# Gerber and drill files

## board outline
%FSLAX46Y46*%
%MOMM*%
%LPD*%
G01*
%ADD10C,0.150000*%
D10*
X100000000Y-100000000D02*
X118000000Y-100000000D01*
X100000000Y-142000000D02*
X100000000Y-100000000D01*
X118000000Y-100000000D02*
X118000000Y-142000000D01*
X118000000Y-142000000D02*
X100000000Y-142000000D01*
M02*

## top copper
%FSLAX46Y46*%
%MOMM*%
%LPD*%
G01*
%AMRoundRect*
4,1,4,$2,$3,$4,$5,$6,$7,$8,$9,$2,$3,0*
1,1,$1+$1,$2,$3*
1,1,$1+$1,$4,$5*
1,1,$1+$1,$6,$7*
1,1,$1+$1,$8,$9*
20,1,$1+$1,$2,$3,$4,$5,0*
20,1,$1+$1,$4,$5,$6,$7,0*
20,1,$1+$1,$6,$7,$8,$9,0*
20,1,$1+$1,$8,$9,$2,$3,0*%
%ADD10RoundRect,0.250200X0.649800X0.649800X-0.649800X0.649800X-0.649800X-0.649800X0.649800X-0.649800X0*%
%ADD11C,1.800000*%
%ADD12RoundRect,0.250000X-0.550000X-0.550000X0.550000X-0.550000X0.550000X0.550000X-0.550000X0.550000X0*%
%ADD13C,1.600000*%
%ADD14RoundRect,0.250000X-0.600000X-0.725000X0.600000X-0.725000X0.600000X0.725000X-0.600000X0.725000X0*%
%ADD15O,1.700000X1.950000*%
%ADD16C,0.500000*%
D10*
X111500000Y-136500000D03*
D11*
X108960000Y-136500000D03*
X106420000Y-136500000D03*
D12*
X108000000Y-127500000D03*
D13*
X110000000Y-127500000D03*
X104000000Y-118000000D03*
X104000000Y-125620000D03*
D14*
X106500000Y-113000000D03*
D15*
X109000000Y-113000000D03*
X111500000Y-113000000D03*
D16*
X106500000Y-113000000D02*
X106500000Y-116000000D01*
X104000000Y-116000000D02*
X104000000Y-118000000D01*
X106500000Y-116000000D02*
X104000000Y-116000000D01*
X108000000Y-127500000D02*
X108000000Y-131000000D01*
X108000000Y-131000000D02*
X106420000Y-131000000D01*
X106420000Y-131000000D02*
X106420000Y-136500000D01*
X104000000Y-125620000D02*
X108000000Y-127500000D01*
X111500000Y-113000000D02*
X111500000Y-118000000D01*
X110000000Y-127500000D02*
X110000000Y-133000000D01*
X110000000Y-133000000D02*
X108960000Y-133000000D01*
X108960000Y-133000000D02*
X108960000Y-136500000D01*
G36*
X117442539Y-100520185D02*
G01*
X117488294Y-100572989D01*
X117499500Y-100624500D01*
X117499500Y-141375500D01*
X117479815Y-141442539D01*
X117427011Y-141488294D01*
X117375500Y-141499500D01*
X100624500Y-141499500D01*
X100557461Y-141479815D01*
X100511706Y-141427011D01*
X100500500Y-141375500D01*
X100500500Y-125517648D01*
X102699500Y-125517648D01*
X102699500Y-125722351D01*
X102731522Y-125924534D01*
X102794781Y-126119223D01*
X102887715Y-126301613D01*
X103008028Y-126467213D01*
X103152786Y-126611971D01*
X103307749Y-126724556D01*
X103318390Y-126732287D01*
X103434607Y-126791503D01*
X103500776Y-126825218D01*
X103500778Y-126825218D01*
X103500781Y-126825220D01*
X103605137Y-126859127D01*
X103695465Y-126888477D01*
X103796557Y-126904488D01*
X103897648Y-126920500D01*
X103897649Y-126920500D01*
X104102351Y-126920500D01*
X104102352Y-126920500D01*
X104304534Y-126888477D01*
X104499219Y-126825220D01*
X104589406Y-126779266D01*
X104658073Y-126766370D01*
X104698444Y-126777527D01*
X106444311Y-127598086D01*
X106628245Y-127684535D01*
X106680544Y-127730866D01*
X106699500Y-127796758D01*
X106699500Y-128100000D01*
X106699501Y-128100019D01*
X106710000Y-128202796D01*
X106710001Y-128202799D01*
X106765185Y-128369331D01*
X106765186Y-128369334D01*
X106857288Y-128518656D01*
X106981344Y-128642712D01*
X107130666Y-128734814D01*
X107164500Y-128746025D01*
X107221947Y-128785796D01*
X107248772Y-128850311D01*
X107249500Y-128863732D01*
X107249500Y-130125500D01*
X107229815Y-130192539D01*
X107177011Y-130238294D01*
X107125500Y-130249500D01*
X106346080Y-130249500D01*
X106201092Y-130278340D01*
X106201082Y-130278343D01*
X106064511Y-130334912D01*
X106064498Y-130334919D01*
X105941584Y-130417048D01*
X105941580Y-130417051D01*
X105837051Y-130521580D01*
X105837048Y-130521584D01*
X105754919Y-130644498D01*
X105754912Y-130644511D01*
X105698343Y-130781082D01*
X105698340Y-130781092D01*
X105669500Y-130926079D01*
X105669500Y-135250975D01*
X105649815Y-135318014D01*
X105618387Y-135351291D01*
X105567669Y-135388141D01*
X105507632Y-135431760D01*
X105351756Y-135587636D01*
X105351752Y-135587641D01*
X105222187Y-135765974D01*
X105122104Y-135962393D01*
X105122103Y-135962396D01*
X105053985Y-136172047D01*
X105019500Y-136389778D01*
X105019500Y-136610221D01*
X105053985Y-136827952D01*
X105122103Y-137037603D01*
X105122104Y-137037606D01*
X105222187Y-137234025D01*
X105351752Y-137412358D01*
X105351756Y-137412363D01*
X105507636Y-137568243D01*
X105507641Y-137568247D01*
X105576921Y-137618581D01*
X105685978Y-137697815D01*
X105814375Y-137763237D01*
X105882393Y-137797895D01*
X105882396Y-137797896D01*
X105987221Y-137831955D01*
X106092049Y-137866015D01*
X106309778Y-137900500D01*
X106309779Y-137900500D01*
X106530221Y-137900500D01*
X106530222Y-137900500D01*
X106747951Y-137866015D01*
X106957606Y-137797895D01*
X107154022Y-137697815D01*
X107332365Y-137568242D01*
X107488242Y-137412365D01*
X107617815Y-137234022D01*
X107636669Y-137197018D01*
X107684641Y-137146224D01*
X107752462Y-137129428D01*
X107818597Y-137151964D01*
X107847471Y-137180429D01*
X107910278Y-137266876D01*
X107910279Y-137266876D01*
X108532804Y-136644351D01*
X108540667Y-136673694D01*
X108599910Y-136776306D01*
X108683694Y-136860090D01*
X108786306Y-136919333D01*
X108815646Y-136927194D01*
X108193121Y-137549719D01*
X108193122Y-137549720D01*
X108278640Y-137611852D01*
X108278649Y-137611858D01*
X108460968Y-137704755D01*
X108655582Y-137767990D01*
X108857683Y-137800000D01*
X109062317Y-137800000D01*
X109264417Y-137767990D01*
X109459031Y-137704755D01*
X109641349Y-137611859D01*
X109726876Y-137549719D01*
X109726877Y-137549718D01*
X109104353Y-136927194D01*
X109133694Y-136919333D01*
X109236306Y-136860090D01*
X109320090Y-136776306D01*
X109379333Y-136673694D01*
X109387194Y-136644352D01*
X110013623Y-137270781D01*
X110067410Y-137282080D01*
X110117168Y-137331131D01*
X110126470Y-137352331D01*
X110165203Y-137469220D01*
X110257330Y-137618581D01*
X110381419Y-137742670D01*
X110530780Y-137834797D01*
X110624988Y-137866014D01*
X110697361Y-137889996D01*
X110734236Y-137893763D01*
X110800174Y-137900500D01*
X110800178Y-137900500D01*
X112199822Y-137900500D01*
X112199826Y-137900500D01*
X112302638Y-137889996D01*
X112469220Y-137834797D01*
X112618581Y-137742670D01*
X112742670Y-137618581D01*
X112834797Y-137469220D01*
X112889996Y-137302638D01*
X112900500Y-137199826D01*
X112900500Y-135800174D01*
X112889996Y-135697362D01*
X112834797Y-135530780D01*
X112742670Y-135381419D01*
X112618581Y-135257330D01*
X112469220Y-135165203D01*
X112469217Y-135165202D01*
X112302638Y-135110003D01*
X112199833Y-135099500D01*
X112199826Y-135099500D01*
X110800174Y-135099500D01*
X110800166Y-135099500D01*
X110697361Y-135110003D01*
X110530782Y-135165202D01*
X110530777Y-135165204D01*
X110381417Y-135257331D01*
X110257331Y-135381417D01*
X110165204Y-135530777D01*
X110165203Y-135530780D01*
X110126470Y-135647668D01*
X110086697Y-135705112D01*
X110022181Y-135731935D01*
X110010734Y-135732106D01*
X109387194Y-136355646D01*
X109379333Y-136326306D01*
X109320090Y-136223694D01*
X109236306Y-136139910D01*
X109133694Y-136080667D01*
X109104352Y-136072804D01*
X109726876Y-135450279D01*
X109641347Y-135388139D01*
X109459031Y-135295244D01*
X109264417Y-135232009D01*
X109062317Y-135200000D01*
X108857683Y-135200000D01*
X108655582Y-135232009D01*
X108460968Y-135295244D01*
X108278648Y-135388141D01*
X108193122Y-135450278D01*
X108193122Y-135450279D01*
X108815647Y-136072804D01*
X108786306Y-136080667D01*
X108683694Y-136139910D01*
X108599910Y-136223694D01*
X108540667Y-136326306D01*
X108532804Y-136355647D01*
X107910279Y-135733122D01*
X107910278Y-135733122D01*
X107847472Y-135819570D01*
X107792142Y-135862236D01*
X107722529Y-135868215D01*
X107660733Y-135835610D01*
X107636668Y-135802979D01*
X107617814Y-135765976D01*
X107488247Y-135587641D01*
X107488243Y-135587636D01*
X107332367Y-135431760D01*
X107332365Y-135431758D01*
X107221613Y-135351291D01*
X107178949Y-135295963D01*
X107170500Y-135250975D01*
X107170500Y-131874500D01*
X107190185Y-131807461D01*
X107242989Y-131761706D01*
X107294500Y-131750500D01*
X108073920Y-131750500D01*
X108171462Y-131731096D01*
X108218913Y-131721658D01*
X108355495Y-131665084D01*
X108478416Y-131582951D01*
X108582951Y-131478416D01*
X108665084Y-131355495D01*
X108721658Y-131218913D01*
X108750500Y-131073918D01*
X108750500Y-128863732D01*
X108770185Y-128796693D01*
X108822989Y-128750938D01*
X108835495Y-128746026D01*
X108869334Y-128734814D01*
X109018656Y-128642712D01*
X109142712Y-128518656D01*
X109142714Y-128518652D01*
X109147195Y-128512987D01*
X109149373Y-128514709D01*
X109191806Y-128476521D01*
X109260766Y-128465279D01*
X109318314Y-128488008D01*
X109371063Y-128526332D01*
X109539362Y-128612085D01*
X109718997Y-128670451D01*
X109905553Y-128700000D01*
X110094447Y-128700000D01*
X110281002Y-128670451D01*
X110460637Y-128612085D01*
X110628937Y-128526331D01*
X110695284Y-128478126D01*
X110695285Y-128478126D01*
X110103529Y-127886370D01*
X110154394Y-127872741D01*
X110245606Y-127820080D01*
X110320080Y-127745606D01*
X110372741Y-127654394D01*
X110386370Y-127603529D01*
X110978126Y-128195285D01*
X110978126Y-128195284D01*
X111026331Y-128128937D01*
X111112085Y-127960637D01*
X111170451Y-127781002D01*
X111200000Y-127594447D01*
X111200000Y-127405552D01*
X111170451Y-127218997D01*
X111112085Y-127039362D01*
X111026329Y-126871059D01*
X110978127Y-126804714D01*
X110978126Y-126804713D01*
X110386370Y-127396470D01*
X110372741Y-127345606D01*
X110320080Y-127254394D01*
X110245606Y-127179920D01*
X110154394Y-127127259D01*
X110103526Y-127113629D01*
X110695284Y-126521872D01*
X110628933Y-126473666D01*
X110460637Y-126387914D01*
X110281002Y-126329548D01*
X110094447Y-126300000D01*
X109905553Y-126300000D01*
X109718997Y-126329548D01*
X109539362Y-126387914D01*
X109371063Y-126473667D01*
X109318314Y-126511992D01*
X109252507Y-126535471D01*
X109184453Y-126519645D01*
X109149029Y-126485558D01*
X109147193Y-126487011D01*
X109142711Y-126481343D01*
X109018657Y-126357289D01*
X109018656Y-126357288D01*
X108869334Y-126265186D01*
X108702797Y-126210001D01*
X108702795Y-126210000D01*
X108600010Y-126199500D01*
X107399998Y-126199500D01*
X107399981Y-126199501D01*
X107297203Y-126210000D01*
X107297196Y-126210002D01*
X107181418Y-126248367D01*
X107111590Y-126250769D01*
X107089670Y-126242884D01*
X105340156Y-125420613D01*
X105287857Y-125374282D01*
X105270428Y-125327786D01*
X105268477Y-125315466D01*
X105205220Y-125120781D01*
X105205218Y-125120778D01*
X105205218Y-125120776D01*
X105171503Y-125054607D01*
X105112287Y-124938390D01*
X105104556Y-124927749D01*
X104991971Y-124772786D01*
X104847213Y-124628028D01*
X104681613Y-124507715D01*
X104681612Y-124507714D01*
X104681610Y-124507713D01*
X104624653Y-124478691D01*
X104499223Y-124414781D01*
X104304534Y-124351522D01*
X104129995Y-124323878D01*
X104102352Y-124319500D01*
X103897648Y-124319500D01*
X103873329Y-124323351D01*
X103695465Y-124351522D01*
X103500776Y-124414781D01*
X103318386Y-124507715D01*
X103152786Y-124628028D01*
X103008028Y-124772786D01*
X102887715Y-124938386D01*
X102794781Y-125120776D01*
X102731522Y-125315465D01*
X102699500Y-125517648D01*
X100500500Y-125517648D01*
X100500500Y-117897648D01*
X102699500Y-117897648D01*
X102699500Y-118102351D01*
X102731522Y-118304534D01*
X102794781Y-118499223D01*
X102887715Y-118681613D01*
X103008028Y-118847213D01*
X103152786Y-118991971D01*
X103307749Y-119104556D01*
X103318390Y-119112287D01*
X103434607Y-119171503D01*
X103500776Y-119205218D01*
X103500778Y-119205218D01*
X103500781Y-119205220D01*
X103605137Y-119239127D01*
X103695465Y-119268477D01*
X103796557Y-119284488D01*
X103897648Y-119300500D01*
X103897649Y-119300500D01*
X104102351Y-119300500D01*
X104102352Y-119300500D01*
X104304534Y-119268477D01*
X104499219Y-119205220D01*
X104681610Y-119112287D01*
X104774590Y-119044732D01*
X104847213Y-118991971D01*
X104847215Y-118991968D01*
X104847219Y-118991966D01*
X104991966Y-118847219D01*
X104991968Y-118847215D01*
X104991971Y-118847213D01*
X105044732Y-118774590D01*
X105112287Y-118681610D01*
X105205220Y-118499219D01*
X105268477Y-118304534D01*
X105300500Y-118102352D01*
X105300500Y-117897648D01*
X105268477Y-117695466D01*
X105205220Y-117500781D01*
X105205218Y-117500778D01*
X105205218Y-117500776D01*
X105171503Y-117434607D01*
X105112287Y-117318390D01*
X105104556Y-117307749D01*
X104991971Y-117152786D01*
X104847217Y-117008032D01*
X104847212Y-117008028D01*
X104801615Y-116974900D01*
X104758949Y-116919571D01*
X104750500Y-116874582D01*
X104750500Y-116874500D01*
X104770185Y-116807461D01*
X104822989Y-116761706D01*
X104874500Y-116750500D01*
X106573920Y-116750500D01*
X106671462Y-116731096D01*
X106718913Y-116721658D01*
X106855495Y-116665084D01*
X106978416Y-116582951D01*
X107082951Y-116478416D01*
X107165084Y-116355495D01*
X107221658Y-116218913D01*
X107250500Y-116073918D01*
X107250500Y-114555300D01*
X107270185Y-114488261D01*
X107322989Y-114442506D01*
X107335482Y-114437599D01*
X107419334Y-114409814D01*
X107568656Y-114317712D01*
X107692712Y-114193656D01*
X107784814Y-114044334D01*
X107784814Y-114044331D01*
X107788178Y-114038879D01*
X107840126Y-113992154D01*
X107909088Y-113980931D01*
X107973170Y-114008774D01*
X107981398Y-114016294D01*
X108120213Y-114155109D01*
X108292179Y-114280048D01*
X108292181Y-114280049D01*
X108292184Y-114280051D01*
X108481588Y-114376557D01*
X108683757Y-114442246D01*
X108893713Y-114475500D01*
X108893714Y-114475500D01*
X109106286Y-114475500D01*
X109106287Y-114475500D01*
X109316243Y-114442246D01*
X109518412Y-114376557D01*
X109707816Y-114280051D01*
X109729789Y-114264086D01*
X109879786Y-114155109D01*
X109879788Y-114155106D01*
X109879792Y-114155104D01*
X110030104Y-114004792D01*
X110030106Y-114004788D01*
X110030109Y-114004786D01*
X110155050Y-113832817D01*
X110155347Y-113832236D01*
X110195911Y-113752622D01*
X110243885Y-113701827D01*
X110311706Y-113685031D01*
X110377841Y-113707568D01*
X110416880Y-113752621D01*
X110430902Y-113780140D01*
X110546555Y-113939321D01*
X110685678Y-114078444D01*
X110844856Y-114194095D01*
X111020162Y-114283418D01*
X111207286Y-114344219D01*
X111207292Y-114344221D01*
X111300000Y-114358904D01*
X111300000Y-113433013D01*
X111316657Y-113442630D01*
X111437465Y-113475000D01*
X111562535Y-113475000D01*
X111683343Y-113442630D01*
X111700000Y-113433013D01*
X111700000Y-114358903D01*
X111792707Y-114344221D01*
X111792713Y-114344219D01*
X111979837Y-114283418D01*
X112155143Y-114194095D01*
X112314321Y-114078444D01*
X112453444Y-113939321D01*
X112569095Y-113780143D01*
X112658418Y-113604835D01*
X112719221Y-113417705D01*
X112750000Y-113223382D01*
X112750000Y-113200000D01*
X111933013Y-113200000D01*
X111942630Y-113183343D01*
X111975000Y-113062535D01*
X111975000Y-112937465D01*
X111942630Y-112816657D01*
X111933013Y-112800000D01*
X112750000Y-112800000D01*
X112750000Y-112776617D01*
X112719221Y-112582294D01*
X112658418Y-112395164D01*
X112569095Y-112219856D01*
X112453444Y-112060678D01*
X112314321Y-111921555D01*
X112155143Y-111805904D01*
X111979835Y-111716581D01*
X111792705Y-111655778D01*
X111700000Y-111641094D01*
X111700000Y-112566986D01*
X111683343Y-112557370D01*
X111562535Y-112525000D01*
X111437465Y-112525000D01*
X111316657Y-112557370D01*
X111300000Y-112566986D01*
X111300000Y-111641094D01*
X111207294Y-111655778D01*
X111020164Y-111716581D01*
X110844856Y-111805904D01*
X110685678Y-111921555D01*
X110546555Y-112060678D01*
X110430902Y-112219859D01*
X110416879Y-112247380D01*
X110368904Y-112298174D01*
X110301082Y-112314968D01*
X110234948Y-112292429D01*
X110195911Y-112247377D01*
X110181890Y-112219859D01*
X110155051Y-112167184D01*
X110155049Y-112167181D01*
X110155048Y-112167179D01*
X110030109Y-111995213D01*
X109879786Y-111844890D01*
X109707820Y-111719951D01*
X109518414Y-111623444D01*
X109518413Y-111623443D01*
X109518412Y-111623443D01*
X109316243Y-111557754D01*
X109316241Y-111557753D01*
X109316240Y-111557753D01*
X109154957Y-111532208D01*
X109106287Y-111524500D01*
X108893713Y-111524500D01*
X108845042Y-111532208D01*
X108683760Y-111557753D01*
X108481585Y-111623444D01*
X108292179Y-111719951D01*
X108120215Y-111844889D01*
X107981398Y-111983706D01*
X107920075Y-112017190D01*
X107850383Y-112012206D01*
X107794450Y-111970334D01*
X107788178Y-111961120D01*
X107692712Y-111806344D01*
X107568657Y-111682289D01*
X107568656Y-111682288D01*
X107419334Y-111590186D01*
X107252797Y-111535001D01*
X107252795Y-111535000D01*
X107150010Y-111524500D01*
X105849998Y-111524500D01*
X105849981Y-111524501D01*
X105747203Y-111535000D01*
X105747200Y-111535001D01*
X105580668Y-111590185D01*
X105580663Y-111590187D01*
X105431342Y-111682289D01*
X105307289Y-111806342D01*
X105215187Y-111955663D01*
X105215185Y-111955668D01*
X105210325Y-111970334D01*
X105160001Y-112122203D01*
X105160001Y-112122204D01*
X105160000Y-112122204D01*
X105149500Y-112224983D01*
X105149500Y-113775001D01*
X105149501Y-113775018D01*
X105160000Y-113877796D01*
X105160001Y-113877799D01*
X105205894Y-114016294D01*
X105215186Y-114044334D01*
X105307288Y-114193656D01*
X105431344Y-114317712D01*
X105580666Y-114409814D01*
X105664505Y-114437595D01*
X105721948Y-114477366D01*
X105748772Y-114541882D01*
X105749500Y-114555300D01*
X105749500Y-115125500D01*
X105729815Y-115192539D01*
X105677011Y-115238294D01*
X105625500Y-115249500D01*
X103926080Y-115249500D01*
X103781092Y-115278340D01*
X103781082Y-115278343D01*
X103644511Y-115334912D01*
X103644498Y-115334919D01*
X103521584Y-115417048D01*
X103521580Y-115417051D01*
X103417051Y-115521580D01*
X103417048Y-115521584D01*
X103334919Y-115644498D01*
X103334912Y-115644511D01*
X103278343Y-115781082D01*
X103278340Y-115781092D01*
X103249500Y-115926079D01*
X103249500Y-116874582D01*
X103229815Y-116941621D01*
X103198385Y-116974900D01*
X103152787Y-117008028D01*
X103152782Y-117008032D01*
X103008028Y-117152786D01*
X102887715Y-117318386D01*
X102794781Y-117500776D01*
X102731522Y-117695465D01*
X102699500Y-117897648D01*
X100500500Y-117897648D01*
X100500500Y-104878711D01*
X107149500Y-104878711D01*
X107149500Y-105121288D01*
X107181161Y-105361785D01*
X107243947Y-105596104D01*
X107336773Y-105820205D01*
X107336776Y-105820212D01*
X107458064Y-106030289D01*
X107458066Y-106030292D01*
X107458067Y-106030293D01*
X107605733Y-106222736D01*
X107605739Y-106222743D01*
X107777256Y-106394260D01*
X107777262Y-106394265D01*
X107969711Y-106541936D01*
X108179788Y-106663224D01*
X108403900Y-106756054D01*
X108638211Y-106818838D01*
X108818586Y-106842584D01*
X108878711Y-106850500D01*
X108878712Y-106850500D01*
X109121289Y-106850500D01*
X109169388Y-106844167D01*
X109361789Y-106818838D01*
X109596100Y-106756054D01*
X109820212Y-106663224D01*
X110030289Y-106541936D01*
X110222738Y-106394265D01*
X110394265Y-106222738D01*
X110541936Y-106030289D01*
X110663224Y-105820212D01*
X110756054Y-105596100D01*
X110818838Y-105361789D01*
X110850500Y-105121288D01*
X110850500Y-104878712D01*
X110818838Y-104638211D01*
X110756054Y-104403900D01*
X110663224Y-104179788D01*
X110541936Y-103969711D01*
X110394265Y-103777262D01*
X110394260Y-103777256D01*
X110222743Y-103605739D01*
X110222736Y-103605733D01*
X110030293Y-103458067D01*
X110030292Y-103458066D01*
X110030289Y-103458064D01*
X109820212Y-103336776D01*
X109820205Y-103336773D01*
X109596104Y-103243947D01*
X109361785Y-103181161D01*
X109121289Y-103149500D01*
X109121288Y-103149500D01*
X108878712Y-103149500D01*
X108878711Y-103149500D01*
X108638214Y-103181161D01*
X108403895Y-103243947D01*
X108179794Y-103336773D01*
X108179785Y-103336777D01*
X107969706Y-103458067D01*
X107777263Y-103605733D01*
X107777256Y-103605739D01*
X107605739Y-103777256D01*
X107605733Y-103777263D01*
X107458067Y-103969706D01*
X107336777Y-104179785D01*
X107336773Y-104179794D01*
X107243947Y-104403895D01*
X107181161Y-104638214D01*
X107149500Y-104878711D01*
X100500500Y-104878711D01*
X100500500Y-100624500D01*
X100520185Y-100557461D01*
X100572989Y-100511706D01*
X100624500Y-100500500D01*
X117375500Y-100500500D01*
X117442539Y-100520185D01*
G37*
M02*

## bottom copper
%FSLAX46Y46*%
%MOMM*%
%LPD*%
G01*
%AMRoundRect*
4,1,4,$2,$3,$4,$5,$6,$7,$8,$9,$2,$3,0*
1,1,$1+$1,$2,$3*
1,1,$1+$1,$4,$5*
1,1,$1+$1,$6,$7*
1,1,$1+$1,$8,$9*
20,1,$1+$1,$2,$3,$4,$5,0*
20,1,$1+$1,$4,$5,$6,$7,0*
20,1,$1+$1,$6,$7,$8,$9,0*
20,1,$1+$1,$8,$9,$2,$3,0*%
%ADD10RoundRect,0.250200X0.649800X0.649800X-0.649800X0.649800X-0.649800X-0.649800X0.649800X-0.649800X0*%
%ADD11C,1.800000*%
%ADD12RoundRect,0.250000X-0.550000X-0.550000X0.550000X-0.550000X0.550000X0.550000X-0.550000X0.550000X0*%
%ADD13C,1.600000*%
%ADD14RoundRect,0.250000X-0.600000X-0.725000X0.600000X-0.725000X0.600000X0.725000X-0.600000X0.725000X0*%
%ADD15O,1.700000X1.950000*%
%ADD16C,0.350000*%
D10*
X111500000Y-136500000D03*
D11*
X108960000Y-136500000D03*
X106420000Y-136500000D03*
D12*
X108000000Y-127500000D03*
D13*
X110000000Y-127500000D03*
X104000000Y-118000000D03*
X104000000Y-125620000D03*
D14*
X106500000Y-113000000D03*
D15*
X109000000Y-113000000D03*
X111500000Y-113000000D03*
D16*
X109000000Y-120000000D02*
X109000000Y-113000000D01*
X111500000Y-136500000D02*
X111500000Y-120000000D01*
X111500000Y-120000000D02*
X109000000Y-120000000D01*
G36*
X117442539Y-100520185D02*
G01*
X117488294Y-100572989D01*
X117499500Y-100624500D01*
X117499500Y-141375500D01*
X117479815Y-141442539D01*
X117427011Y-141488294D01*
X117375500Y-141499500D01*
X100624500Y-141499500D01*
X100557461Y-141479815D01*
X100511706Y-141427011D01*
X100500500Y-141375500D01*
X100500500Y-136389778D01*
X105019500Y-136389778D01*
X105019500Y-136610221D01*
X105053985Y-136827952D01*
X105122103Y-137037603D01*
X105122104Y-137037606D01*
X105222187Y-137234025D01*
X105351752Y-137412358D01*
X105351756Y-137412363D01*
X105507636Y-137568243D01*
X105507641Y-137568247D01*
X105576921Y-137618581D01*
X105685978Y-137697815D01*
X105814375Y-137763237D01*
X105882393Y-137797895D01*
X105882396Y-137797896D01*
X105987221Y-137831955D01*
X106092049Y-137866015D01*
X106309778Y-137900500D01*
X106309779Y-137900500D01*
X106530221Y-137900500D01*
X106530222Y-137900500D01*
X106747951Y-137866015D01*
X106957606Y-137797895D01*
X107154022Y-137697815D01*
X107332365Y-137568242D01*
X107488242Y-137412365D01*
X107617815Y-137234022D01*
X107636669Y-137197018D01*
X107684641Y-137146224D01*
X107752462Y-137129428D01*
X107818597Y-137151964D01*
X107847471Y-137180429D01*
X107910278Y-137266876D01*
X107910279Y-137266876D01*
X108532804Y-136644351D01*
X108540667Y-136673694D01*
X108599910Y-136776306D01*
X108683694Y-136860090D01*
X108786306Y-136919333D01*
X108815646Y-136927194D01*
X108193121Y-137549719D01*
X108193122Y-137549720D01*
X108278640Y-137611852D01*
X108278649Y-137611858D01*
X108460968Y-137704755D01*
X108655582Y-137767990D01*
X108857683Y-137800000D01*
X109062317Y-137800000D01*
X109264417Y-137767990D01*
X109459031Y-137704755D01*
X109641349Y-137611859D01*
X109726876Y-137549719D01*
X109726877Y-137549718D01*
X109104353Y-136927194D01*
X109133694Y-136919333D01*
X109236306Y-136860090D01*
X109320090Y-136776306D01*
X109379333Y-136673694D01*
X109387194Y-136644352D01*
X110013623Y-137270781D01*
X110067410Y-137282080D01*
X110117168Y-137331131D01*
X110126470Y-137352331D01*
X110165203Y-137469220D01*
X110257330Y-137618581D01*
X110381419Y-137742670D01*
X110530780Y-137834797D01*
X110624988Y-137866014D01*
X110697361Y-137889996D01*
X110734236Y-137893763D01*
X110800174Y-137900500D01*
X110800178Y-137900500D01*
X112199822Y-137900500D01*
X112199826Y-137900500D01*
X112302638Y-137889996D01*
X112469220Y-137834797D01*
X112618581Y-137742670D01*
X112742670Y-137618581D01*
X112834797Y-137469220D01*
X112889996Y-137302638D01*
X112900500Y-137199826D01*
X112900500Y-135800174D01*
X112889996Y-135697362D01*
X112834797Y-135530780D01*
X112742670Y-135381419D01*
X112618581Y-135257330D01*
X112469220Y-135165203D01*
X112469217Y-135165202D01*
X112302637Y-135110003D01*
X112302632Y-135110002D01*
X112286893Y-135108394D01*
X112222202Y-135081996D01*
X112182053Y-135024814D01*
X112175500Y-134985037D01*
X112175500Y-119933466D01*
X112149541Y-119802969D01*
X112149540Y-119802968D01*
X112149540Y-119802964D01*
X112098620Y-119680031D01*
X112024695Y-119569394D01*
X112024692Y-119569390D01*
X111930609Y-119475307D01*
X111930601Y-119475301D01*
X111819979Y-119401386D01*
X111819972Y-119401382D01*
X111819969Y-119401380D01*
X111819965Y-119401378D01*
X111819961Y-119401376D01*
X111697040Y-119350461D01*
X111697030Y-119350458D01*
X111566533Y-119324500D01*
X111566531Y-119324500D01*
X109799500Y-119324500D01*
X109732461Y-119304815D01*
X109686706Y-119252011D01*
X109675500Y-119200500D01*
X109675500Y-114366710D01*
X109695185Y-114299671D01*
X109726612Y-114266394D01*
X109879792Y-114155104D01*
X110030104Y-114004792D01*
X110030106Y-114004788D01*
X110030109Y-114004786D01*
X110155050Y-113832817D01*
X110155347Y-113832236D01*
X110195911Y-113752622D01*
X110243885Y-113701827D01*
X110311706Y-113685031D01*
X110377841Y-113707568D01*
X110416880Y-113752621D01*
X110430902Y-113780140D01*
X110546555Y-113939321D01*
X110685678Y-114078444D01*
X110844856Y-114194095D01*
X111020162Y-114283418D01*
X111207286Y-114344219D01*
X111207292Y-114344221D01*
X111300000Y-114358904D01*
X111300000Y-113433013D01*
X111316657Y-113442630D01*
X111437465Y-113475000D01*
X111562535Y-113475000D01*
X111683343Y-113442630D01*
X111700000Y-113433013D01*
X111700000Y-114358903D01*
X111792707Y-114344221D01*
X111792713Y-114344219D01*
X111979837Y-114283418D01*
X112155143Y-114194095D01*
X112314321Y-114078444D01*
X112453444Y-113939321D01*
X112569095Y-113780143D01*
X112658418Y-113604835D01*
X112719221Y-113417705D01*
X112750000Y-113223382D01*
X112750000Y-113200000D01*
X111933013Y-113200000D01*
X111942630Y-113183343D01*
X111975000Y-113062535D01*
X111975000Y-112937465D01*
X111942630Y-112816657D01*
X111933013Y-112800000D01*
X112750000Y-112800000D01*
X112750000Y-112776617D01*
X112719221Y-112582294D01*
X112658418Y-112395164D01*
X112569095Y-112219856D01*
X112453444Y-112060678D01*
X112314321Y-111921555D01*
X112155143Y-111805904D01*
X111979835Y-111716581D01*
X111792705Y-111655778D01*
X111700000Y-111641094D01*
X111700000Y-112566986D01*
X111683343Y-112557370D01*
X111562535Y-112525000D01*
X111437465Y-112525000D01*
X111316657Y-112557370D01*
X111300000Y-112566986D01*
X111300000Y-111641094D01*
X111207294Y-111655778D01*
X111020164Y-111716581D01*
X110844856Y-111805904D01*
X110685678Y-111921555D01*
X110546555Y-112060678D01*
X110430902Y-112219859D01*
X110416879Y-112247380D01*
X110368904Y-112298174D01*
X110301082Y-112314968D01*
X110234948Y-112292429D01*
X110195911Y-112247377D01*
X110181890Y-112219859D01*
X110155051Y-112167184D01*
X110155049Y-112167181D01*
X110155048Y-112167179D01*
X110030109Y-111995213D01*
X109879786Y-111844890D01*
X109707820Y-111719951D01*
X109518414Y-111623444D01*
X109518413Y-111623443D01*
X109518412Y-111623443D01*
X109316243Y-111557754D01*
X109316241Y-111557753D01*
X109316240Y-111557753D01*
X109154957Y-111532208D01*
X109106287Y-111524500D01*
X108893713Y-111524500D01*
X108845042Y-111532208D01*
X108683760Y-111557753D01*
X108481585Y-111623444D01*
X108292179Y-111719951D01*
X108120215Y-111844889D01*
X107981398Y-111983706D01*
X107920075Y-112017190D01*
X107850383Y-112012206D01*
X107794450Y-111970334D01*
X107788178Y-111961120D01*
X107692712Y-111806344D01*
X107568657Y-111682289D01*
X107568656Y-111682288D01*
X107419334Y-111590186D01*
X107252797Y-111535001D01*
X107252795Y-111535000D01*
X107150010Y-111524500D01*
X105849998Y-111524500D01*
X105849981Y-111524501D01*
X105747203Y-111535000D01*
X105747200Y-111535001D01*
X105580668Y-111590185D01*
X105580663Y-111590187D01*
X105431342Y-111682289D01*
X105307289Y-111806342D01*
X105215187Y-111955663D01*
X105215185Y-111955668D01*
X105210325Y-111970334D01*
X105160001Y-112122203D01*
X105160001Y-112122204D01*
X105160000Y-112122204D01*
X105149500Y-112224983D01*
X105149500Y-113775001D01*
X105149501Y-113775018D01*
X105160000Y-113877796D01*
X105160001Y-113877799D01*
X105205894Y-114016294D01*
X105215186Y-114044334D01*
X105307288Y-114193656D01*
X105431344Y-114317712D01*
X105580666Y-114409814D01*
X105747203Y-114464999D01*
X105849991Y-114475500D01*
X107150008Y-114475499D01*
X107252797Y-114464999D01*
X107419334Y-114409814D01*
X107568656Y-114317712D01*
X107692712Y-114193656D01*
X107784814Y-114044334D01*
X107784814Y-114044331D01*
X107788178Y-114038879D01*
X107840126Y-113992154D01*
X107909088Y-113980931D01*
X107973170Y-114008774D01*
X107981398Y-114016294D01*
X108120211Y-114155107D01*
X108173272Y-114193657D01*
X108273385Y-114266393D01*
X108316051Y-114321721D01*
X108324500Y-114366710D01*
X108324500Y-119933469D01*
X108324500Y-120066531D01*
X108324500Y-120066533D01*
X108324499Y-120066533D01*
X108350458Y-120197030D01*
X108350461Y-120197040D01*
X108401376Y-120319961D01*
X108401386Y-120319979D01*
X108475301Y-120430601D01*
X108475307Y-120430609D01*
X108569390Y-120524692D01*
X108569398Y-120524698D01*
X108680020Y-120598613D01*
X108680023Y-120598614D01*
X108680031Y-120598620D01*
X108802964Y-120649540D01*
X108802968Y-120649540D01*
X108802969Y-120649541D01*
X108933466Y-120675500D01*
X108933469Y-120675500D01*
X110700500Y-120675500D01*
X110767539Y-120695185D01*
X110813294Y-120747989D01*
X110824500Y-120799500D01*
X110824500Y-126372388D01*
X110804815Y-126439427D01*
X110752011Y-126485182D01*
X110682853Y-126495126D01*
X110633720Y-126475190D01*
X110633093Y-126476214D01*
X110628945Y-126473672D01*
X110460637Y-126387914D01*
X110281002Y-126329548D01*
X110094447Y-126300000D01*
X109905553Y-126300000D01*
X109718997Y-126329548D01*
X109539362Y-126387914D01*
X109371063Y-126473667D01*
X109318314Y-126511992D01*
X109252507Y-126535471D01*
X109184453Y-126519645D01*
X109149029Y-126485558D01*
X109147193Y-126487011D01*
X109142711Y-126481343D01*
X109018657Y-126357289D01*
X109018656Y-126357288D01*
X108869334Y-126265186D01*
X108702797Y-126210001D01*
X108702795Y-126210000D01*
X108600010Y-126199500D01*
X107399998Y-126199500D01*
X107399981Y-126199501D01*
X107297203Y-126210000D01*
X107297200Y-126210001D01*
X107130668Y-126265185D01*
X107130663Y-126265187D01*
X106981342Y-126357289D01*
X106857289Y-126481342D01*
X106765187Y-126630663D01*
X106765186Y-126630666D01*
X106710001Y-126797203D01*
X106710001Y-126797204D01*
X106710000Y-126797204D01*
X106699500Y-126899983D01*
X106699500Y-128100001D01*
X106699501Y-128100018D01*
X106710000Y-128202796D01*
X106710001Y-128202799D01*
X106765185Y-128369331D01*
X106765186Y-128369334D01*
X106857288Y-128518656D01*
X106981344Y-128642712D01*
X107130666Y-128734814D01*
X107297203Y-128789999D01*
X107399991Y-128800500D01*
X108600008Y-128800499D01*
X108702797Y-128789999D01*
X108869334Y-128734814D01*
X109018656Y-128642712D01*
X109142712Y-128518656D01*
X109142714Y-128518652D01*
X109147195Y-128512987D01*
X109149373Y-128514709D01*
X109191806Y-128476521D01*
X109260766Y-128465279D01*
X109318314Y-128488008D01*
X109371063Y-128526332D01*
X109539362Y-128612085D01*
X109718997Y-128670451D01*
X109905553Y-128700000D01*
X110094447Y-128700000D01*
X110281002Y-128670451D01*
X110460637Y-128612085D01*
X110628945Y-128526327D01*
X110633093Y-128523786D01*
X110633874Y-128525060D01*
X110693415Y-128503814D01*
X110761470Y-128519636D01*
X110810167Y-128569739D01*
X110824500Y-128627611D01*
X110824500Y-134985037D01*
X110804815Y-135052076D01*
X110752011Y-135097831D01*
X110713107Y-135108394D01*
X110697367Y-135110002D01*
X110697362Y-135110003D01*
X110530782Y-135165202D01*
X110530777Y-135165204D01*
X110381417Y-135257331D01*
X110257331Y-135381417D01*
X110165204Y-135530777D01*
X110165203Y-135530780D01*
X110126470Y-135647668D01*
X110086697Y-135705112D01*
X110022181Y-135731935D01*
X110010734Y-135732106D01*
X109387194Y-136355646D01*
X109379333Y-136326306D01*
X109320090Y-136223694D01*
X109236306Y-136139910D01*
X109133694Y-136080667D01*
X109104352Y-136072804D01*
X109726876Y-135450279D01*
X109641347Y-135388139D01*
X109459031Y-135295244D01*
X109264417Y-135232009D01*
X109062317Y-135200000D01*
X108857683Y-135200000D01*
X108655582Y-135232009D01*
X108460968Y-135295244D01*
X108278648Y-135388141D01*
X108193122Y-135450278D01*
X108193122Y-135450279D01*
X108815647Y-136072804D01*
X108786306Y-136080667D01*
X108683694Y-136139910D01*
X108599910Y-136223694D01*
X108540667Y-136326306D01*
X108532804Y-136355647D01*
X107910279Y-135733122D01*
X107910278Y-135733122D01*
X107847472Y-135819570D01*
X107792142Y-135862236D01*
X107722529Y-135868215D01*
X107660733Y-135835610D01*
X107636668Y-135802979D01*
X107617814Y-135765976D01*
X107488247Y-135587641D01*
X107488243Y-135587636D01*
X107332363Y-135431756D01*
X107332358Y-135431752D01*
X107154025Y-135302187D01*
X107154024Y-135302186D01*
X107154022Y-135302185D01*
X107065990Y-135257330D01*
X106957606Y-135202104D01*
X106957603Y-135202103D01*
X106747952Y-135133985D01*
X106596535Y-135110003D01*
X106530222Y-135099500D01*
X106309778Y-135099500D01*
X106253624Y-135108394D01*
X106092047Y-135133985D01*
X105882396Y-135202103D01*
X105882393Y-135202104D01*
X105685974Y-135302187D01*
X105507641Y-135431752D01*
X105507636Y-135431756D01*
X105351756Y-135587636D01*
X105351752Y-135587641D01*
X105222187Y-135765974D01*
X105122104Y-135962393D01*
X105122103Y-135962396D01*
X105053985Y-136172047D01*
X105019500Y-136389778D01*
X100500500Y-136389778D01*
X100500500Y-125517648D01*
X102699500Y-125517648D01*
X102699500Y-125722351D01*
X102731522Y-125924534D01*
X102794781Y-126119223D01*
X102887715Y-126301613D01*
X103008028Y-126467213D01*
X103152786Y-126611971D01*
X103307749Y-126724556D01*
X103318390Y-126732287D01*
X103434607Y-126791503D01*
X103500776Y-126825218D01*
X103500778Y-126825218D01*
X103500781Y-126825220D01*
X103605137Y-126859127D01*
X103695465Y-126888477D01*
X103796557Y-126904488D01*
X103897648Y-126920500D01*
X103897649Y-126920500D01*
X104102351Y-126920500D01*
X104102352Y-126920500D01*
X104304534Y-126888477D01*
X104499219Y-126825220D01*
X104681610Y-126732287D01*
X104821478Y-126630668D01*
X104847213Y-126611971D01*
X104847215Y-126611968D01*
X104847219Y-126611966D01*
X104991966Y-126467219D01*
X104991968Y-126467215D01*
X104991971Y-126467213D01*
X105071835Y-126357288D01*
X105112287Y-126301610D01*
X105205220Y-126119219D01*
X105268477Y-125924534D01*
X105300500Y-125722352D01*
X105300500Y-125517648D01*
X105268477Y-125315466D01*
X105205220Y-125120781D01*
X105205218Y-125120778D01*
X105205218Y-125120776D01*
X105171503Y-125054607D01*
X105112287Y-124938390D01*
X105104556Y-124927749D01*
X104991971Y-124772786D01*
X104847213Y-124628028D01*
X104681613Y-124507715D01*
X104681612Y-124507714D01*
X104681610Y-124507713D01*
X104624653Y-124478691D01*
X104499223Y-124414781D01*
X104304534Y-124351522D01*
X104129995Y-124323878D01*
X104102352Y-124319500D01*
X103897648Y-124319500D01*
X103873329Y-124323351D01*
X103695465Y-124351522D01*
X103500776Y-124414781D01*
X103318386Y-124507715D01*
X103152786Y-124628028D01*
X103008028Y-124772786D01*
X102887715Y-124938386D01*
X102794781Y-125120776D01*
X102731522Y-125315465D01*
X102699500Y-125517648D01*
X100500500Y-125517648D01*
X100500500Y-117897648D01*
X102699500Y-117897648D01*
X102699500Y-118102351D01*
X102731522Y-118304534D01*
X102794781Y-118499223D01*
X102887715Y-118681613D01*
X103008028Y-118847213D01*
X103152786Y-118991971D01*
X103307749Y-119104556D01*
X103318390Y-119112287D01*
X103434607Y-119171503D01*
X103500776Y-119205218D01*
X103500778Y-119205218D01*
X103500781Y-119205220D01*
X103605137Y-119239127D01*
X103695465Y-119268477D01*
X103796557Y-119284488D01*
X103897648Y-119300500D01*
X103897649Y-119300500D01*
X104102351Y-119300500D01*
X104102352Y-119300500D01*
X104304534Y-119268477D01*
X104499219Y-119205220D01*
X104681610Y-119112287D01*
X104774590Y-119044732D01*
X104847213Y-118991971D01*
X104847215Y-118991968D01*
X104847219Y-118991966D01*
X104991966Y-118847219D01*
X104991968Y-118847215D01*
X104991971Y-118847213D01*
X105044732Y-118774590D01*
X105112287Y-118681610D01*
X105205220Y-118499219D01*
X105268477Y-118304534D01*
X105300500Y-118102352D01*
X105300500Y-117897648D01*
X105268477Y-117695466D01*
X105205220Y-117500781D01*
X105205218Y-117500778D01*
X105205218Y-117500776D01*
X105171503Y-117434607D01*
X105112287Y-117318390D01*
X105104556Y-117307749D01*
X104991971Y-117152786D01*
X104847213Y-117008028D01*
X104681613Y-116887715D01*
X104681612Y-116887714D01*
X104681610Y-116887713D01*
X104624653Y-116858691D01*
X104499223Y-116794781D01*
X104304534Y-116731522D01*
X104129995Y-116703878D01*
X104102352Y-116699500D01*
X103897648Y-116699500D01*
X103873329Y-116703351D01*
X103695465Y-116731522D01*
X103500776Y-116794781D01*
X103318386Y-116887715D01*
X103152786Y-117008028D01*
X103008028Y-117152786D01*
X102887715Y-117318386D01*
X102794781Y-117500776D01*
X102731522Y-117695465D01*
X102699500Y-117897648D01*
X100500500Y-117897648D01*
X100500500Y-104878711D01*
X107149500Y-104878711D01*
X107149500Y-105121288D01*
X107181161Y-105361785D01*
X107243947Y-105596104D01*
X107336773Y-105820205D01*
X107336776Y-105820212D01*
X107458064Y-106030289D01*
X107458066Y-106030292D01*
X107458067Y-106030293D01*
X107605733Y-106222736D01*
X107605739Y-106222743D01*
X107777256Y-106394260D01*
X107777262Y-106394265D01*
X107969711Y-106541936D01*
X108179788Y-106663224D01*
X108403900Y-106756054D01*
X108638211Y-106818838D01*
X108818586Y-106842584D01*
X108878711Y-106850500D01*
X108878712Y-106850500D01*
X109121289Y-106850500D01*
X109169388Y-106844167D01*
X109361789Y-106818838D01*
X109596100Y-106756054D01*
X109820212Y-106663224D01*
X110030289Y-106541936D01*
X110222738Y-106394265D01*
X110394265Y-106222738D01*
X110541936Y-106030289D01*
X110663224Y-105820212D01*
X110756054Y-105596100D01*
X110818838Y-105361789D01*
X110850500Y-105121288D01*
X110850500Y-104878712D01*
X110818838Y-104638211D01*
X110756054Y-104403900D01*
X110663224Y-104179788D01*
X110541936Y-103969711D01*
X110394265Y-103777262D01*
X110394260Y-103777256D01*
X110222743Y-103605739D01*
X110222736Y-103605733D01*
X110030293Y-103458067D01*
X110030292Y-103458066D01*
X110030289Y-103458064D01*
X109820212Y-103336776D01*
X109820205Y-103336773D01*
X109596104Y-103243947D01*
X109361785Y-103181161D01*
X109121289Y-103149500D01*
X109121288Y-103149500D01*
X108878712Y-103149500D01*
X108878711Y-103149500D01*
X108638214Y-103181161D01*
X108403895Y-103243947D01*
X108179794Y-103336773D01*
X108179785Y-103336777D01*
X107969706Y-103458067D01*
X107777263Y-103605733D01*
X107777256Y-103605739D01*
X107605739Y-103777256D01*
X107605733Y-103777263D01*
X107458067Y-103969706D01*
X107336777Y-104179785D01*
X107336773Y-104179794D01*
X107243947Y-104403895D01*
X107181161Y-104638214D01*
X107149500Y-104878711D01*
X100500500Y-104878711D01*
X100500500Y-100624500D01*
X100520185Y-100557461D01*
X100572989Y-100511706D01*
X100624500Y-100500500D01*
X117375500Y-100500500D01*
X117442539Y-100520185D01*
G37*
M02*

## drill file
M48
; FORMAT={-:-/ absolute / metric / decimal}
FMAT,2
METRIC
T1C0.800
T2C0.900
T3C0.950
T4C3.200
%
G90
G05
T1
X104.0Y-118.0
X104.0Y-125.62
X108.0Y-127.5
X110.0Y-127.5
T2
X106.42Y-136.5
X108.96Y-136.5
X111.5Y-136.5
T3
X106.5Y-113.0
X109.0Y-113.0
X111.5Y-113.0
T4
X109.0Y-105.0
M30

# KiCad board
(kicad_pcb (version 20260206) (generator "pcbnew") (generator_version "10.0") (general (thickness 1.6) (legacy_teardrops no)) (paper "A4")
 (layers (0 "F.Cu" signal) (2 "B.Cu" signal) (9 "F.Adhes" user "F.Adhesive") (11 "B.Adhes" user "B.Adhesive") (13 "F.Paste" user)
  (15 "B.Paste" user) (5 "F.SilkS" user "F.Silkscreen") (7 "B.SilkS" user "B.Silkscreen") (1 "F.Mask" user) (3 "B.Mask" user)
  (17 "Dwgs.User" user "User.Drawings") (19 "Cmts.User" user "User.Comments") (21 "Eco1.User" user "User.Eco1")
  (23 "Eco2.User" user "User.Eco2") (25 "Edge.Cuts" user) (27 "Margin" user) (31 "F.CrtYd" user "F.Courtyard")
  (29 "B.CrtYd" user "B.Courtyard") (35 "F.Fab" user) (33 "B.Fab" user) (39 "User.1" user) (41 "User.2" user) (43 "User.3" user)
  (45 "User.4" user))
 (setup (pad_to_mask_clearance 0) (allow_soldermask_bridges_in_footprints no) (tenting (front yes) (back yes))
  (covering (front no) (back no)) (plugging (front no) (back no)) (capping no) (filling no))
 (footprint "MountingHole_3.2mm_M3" (layer "F.Cu") (at 109 105)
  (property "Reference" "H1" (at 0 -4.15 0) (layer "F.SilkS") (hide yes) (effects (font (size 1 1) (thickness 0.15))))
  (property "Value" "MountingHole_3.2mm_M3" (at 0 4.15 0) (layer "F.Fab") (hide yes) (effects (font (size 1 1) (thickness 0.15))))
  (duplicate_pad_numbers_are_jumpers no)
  (pad "" np_thru_hole circle (at 0 0) (size 3.2 3.2) (drill 3.2) (layers "*.Cu" "*.Mask")))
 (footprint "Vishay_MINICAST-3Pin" (layer "F.Cu") (at 111.5 136.5 180)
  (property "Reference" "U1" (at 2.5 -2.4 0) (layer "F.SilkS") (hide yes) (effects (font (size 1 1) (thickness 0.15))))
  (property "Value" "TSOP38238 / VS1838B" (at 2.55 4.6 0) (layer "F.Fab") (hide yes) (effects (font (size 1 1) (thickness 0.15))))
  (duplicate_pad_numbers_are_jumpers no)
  (pad "1" thru_hole roundrect (at 0 0 180) (size 1.8 1.8) (drill 0.9) (layers "*.Cu" "*.Mask") (remove_unused_layers no)
   (roundrect_rratio 0.139) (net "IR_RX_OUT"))
  (pad "2" thru_hole circle (at 2.54 0 180) (size 1.8 1.8) (drill 0.9) (layers "*.Cu" "*.Mask") (remove_unused_layers no) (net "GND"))
  (pad "3" thru_hole circle (at 5.08 0 180) (size 1.8 1.8) (drill 0.9) (layers "*.Cu" "*.Mask") (remove_unused_layers no) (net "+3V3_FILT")))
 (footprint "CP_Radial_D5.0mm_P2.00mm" (layer "F.Cu") (at 108 127.5)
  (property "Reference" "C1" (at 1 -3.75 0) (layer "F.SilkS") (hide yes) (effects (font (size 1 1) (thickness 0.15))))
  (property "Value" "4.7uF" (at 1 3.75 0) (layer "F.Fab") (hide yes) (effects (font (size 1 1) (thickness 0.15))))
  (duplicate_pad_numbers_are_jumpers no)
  (pad "1" thru_hole roundrect (at 0 0) (size 1.6 1.6) (drill 0.8) (layers "*.Cu" "*.Mask") (remove_unused_layers no)
   (roundrect_rratio 0.15625) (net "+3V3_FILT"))
  (pad "2" thru_hole circle (at 2 0) (size 1.6 1.6) (drill 0.8) (layers "*.Cu" "*.Mask") (remove_unused_layers no) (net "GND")))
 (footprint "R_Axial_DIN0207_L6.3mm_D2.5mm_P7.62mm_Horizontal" (layer "F.Cu") (at 104 118 -90)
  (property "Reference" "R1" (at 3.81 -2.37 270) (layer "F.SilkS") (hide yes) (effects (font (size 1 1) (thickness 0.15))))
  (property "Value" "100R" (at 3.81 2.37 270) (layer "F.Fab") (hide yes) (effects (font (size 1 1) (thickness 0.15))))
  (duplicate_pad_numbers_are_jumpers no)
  (pad "1" thru_hole circle (at 0 0 270) (size 1.6 1.6) (drill 0.8) (layers "*.Cu" "*.Mask") (remove_unused_layers no) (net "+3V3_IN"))
  (pad "2" thru_hole circle (at 7.62 0 270) (size 1.6 1.6) (drill 0.8) (layers "*.Cu" "*.Mask") (remove_unused_layers no) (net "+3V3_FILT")))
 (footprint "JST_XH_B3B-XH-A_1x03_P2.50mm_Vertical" (layer "F.Cu") (at 106.5 113)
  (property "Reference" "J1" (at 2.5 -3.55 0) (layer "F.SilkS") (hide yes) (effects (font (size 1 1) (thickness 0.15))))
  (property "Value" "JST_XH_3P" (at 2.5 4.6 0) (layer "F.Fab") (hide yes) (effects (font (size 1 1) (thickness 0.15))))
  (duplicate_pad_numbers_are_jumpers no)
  (pad "1" thru_hole roundrect (at 0 0) (size 1.7 1.95) (drill 0.95) (layers "*.Cu" "*.Mask") (remove_unused_layers no)
   (roundrect_rratio 0.147059) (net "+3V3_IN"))
  (pad "2" thru_hole oval (at 2.5 0) (size 1.7 1.95) (drill 0.95) (layers "*.Cu" "*.Mask") (remove_unused_layers no) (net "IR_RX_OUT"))
  (pad "3" thru_hole oval (at 5 0) (size 1.7 1.95) (drill 0.95) (layers "*.Cu" "*.Mask") (remove_unused_layers no) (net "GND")))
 (gr_line (start 100 100) (end 118 100) (stroke (width 0.15) (type default)) (layer "Edge.Cuts"))
 (gr_line (start 100 142) (end 100 100) (stroke (width 0.15) (type default)) (layer "Edge.Cuts"))
 (gr_line (start 118 100) (end 118 142) (stroke (width 0.15) (type default)) (layer "Edge.Cuts"))
 (gr_line (start 118 142) (end 100 142) (stroke (width 0.15) (type default)) (layer "Edge.Cuts"))
 (segment (start 106.5 113) (end 106.5 116) (width 0.5) (layer "F.Cu") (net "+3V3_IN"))
 (segment (start 104 116) (end 104 118) (width 0.5) (layer "F.Cu") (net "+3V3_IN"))
 (segment (start 106.5 116) (end 104 116) (width 0.5) (layer "F.Cu") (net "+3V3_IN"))
 (segment (start 108 127.5) (end 108 131) (width 0.5) (layer "F.Cu") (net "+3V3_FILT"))
 (segment (start 108 131) (end 106.42 131) (width 0.5) (layer "F.Cu") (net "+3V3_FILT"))
 (segment (start 106.42 131) (end 106.42 136.5) (width 0.5) (layer "F.Cu") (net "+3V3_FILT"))
 (segment (start 104 125.62) (end 108 127.5) (width 0.5) (layer "F.Cu") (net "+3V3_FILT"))
 (segment (start 109 120) (end 109 113) (width 0.35) (layer "B.Cu") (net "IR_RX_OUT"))
 (segment (start 111.5 136.5) (end 111.5 120) (width 0.35) (layer "B.Cu") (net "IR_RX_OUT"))
 (segment (start 111.5 120) (end 109 120) (width 0.35) (layer "B.Cu") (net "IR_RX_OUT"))
 (segment (start 111.5 113) (end 111.5 118) (width 0.5) (layer "F.Cu") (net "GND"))
 (segment (start 110 127.5) (end 110 133) (width 0.5) (layer "F.Cu") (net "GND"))
 (segment (start 110 133) (end 108.96 133) (width 0.5) (layer "F.Cu") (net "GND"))
 (segment (start 108.96 133) (end 108.96 136.5) (width 0.5) (layer "F.Cu") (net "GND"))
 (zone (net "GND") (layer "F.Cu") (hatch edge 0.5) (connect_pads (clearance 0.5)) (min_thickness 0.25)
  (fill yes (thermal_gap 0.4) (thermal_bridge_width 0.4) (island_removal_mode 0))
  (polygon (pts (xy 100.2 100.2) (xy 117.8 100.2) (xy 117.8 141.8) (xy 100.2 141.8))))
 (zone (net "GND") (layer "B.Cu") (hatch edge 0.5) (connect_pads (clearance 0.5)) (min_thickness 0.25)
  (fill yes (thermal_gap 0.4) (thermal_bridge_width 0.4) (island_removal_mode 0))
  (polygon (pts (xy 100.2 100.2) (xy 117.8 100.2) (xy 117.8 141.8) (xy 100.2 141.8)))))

